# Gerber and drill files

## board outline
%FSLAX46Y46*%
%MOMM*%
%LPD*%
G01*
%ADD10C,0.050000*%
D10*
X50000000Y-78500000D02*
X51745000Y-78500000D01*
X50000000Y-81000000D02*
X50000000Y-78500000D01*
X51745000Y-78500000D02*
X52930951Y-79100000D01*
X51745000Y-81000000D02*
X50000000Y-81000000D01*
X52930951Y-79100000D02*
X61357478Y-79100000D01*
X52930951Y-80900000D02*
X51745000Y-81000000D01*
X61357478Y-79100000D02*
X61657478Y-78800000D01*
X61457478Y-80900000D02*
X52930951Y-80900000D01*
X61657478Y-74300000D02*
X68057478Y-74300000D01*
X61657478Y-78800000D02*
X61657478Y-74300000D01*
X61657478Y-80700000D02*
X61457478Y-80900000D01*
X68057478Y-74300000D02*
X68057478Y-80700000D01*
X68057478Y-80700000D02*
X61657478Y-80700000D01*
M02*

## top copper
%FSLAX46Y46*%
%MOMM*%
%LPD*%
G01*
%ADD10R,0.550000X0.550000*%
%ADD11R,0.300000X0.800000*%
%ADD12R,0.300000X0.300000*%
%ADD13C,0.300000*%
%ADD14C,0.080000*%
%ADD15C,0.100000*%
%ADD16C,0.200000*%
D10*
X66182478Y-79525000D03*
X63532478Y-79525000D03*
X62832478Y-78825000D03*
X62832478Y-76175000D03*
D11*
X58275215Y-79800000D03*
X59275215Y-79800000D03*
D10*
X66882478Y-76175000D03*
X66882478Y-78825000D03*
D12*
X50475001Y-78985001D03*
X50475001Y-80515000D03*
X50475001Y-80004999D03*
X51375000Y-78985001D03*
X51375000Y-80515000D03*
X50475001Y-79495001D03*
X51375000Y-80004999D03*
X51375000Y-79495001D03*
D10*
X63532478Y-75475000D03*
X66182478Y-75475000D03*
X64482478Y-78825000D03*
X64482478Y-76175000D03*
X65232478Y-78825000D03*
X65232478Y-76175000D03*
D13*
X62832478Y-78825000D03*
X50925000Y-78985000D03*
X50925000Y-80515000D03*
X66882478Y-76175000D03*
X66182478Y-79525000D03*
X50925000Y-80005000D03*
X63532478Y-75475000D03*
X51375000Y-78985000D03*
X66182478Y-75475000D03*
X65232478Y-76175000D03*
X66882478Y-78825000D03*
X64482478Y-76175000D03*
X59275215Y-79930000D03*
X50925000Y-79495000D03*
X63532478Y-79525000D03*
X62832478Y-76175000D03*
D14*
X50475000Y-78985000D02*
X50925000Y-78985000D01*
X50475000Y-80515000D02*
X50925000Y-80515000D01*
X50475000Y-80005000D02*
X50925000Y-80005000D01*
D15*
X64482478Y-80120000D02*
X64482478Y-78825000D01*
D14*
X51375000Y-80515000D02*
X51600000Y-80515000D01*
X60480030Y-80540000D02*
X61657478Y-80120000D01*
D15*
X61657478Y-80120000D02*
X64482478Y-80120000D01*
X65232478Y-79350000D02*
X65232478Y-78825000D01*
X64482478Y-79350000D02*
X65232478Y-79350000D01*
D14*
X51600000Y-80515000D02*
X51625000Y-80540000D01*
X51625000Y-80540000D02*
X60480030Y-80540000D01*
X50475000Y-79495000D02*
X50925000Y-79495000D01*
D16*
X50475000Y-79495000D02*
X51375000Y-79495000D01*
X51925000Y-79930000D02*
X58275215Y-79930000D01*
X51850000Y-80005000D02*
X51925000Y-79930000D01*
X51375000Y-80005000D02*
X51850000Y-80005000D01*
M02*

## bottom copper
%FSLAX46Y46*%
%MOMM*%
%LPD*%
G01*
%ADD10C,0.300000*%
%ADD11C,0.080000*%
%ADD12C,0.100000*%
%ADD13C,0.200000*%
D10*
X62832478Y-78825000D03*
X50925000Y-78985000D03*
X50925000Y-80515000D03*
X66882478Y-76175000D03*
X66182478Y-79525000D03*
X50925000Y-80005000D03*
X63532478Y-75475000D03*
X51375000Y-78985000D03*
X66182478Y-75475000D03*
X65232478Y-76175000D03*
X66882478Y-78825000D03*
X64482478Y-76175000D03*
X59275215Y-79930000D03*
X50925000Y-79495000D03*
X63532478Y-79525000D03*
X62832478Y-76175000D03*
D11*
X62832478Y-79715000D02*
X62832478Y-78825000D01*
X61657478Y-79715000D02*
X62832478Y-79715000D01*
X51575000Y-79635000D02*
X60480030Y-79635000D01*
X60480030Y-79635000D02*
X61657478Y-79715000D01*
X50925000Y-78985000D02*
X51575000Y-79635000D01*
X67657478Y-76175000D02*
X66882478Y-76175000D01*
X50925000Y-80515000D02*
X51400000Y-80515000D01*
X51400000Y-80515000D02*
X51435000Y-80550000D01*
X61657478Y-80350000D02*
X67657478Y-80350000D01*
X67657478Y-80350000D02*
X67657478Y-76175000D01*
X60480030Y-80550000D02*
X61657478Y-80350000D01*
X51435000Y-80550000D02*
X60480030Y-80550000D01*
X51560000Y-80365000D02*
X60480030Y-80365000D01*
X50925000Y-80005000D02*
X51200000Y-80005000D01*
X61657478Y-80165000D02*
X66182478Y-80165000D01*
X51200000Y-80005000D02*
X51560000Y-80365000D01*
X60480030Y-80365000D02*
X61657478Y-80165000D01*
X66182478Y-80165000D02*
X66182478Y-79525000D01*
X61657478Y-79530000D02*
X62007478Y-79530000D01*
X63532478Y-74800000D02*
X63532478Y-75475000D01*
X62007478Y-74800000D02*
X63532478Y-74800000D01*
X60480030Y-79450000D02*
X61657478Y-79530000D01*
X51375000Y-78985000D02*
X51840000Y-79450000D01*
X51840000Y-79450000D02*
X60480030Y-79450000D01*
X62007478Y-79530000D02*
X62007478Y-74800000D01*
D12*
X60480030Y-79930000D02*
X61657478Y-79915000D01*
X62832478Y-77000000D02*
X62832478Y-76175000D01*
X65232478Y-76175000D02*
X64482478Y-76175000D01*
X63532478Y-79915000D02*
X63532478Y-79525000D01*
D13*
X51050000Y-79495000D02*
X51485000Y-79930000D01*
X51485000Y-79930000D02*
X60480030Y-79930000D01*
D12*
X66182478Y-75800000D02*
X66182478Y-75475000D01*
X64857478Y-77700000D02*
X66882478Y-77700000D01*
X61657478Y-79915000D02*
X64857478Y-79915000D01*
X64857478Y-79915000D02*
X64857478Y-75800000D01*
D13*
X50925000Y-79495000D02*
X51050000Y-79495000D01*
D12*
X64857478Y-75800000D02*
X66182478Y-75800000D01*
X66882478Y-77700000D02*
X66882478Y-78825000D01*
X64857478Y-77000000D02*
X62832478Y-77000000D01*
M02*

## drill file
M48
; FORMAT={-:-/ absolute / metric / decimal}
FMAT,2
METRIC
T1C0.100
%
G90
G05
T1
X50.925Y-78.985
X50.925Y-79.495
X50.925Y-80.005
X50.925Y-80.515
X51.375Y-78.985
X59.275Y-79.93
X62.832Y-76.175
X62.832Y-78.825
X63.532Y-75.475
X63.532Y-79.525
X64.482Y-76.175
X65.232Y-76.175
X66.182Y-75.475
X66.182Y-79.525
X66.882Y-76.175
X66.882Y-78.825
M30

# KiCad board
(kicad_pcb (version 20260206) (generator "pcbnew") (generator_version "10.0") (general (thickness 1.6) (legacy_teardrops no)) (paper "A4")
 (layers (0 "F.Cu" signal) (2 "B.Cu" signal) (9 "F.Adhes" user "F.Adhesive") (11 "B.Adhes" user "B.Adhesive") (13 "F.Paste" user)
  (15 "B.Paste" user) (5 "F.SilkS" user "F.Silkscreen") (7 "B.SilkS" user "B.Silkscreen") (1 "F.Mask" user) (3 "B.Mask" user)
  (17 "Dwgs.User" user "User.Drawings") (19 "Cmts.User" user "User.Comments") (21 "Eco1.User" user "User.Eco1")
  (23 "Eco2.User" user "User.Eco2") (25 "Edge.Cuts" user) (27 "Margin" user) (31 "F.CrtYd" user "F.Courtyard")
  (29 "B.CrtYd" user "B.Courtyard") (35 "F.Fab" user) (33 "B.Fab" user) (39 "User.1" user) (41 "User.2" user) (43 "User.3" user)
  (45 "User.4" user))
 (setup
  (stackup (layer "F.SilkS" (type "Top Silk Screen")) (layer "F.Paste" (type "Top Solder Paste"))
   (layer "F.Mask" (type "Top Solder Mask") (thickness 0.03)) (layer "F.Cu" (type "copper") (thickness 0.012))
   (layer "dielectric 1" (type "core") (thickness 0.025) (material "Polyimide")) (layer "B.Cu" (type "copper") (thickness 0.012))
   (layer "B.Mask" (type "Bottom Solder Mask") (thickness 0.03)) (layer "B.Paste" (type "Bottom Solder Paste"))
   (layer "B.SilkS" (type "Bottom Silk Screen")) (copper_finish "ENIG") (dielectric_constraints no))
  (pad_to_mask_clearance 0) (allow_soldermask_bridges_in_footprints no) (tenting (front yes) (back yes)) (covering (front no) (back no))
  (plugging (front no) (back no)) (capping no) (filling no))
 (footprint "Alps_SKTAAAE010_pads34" (layer "F.Cu") (at 64.857478 75.1)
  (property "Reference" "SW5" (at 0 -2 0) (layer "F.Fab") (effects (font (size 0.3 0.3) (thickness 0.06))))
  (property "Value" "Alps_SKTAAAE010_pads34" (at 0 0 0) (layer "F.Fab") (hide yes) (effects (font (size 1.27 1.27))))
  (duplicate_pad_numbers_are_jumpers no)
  (pad "3" smd rect (at -1.325 0.375) (size 0.55 0.55) (layers "F.Cu" "F.Mask" "F.Paste") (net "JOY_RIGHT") (solder_mask_margin 0.05)
   (thermal_bridge_angle 45))
  (pad "4" smd rect (at 1.325 0.375) (size 0.55 0.55) (layers "F.Cu" "F.Mask" "F.Paste") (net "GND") (solder_mask_margin 0.05)
   (thermal_bridge_angle 45)))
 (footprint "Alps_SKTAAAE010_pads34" (layer "F.Cu") (at 62.457478 77.5 90)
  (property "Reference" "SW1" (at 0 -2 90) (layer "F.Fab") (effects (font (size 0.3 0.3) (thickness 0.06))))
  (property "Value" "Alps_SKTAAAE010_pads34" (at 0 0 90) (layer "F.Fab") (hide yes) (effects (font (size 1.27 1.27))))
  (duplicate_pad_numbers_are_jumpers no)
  (pad "3" smd rect (at -1.325 0.375 90) (size 0.55 0.55) (layers "F.Cu" "F.Mask" "F.Paste") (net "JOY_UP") (solder_mask_margin 0.05)
   (thermal_bridge_angle 45))
  (pad "4" smd rect (at 1.325 0.375 90) (size 0.55 0.55) (layers "F.Cu" "F.Mask" "F.Paste") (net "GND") (solder_mask_margin 0.05)
   (thermal_bridge_angle 45)))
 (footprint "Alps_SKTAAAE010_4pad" (layer "F.Cu") (at 64.857478 77.5 90)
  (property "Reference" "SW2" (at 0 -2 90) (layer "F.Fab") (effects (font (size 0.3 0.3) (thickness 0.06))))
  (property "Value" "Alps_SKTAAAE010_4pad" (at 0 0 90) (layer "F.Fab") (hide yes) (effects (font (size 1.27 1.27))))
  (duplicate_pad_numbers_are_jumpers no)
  (pad "1" smd rect (at -1.325 -0.375 90) (size 0.55 0.55) (layers "F.Cu" "F.Mask" "F.Paste") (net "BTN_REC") (solder_mask_margin 0.05)
   (thermal_bridge_angle 45))
  (pad "2" smd rect (at 1.325 -0.375 90) (size 0.55 0.55) (layers "F.Cu" "F.Mask" "F.Paste") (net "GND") (solder_mask_margin 0.05)
   (thermal_bridge_angle 45))
  (pad "3" smd rect (at -1.325 0.375 90) (size 0.55 0.55) (layers "F.Cu" "F.Mask" "F.Paste") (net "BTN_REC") (solder_mask_margin 0.05)
   (thermal_bridge_angle 45))
  (pad "4" smd rect (at 1.325 0.375 90) (size 0.55 0.55) (layers "F.Cu" "F.Mask" "F.Paste") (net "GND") (solder_mask_margin 0.05)
   (thermal_bridge_angle 45)))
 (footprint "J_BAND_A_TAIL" (layer "F.Cu") (at 50.9 79.75)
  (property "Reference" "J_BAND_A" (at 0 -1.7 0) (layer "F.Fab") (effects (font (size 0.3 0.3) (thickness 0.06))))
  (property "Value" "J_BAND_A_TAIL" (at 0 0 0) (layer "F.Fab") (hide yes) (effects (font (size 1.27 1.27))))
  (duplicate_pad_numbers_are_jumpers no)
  (pad "1" smd rect (at -0.424999 -0.764999) (size 0.3 0.3) (layers "F.Cu" "F.Mask") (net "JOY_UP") (solder_mask_margin 0.05)
   (thermal_bridge_angle 45))
  (pad "2" smd rect (at -0.424999 0.765) (size 0.3 0.3) (layers "F.Cu" "F.Mask") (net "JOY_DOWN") (solder_mask_margin 0.05)
   (thermal_bridge_angle 45))
  (pad "3" smd rect (at -0.424999 0.254999) (size 0.3 0.3) (layers "F.Cu" "F.Mask") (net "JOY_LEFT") (solder_mask_margin 0.05)
   (thermal_bridge_angle 45))
  (pad "4" smd rect (at 0.475 -0.764999) (size 0.3 0.3) (layers "F.Cu" "F.Mask") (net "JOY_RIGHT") (solder_mask_margin 0.05)
   (thermal_bridge_angle 45))
  (pad "5" smd rect (at 0.475 0.765) (size 0.3 0.3) (layers "F.Cu" "F.Mask") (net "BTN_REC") (solder_mask_margin 0.05)
   (thermal_bridge_angle 45))
  (pad "6" smd rect (at -0.424999 -0.254999) (size 0.3 0.3) (layers "F.Cu" "F.Mask") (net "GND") (solder_mask_margin 0.05)
   (thermal_bridge_angle 45))
  (pad "7" smd rect (at 0.475 0.254999) (size 0.3 0.3) (layers "F.Cu" "F.Mask") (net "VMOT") (solder_mask_margin 0.05)
   (thermal_bridge_angle 45))
  (pad "8" smd rect (at 0.475 -0.254999) (size 0.3 0.3) (layers "F.Cu" "F.Mask") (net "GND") (solder_mask_margin 0.05)
   (thermal_bridge_angle 45)))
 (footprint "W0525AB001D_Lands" (layer "F.Cu") (at 58.775215 79.93)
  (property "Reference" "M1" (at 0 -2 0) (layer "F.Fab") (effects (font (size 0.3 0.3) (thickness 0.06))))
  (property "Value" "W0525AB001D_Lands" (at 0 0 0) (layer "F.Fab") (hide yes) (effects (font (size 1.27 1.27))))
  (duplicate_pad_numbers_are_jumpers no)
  (pad "1" smd rect (at -0.5 -0.13) (size 0.3 0.8) (layers "F.Cu" "F.Mask") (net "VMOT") (solder_mask_margin 0.05) (thermal_bridge_angle 45))
  (pad "2" smd rect (at 0.5 -0.13) (size 0.3 0.8) (layers "F.Cu" "F.Mask") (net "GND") (solder_mask_margin 0.05) (thermal_bridge_angle 45)))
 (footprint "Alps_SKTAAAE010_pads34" (layer "F.Cu") (at 64.857478 79.9 180)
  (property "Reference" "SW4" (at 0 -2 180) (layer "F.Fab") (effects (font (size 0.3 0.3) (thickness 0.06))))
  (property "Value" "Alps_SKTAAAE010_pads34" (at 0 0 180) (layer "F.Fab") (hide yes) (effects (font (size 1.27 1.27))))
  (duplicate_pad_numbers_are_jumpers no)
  (pad "3" smd rect (at -1.325 0.375 180) (size 0.55 0.55) (layers "F.Cu" "F.Mask" "F.Paste") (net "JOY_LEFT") (solder_mask_margin 0.05)
   (thermal_bridge_angle 45))
  (pad "4" smd rect (at 1.325 0.375 180) (size 0.55 0.55) (layers "F.Cu" "F.Mask" "F.Paste") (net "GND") (solder_mask_margin 0.05)
   (thermal_bridge_angle 45)))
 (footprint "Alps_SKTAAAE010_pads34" (layer "F.Cu") (at 67.257478 77.5 -90)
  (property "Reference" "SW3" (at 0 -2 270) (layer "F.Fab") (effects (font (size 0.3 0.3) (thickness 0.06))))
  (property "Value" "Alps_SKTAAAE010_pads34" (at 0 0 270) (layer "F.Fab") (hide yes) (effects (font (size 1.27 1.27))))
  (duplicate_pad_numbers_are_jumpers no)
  (pad "3" smd rect (at -1.325 0.375 270) (size 0.55 0.55) (layers "F.Cu" "F.Mask" "F.Paste") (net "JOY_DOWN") (solder_mask_margin 0.05)
   (thermal_bridge_angle 45))
  (pad "4" smd rect (at 1.325 0.375 270) (size 0.55 0.55) (layers "F.Cu" "F.Mask" "F.Paste") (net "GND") (solder_mask_margin 0.05)
   (thermal_bridge_angle 45)))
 (gr_line (start 50 78.5) (end 51.745 78.5) (stroke (width 0.05) (type default)) (layer "Edge.Cuts"))
 (gr_line (start 50 81) (end 50 78.5) (stroke (width 0.05) (type default)) (layer "Edge.Cuts"))
 (gr_line (start 51.745 78.5) (end 52.930951 79.1) (stroke (width 0.05) (type default)) (layer "Edge.Cuts"))
 (gr_line (start 51.745 81) (end 50 81) (stroke (width 0.05) (type default)) (layer "Edge.Cuts"))
 (gr_line (start 52.930951 79.1) (end 61.357478 79.1) (stroke (width 0.05) (type default)) (layer "Edge.Cuts"))
 (gr_line (start 52.930951 80.9) (end 51.745 81) (stroke (width 0.05) (type default)) (layer "Edge.Cuts"))
 (gr_line (start 61.357478 79.1) (end 61.657478 78.8) (stroke (width 0.05) (type default)) (layer "Edge.Cuts"))
 (gr_line (start 61.457478 80.9) (end 52.930951 80.9) (stroke (width 0.05) (type default)) (layer "Edge.Cuts"))
 (gr_line (start 61.657478 74.3) (end 68.057478 74.3) (stroke (width 0.05) (type default)) (layer "Edge.Cuts"))
 (gr_line (start 61.657478 78.8) (end 61.657478 74.3) (stroke (width 0.05) (type default)) (layer "Edge.Cuts"))
 (gr_line (start 61.657478 80.7) (end 61.457478 80.9) (stroke (width 0.05) (type default)) (layer "Edge.Cuts"))
 (gr_line (start 68.057478 74.3) (end 68.057478 80.7) (stroke (width 0.05) (type default)) (layer "Edge.Cuts"))
 (gr_line (start 68.057478 80.7) (end 61.657478 80.7) (stroke (width 0.05) (type default)) (layer "Edge.Cuts"))
 (segment (start 50.475 78.985) (end 50.925 78.985) (width 0.08) (layer "F.Cu") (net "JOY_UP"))
 (via (at 50.925 78.985) (size 0.3) (drill 0.1) (layers "F.Cu" "B.Cu") (tenting (front yes) (back yes)) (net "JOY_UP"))
 (via (at 62.832478 78.825) (size 0.3) (drill 0.1) (layers "F.Cu" "B.Cu") (tenting (front yes) (back yes)) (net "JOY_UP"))
 (segment (start 60.48003 79.635) (end 61.657478 79.715) (width 0.08) (layer "B.Cu") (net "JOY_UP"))
 (segment (start 61.657478 79.715) (end 62.832478 79.715) (width 0.08) (layer "B.Cu") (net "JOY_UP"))
 (segment (start 50.925 78.985) (end 51.575 79.635) (width 0.08) (layer "B.Cu") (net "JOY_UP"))
 (segment (start 62.832478 79.715) (end 62.832478 78.825) (width 0.08) (layer "B.Cu") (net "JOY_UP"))
 (segment (start 51.575 79.635) (end 60.48003 79.635) (width 0.08) (layer "B.Cu") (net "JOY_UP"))
 (segment (start 50.475 80.515) (end 50.925 80.515) (width 0.08) (layer "F.Cu") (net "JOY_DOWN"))
 (via (at 50.925 80.515) (size 0.3) (drill 0.1) (layers "F.Cu" "B.Cu") (tenting (front yes) (back yes)) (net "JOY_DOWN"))
 (via (at 66.882478 76.175) (size 0.3) (drill 0.1) (layers "F.Cu" "B.Cu") (tenting (front yes) (back yes)) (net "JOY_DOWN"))
 (segment (start 50.925 80.515) (end 51.4 80.515) (width 0.08) (layer "B.Cu") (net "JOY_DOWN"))
 (segment (start 67.657478 80.35) (end 67.657478 76.175) (width 0.08) (layer "B.Cu") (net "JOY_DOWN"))
 (segment (start 60.48003 80.55) (end 61.657478 80.35) (width 0.08) (layer "B.Cu") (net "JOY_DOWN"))
 (segment (start 67.657478 76.175) (end 66.882478 76.175) (width 0.08) (layer "B.Cu") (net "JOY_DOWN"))
 (segment (start 51.435 80.55) (end 60.48003 80.55) (width 0.08) (layer "B.Cu") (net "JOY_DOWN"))
 (segment (start 51.4 80.515) (end 51.435 80.55) (width 0.08) (layer "B.Cu") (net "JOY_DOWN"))
 (segment (start 61.657478 80.35) (end 67.657478 80.35) (width 0.08) (layer "B.Cu") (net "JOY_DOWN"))
 (segment (start 50.475 80.005) (end 50.925 80.005) (width 0.08) (layer "F.Cu") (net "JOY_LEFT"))
 (via (at 66.182478 79.525) (size 0.3) (drill 0.1) (layers "F.Cu" "B.Cu") (tenting (front yes) (back yes)) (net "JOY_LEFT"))
 (via (at 50.925 80.005) (size 0.3) (drill 0.1) (layers "F.Cu" "B.Cu") (tenting (front yes) (back yes)) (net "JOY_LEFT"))
 (segment (start 51.56 80.365) (end 60.48003 80.365) (width 0.08) (layer "B.Cu") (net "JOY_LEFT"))
 (segment (start 61.657478 80.165) (end 66.182478 80.165) (width 0.08) (layer "B.Cu") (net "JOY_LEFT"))
 (segment (start 51.2 80.005) (end 51.56 80.365) (width 0.08) (layer "B.Cu") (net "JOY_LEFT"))
 (segment (start 60.48003 80.365) (end 61.657478 80.165) (width 0.08) (layer "B.Cu") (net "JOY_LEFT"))
 (segment (start 66.182478 80.165) (end 66.182478 79.525) (width 0.08) (layer "B.Cu") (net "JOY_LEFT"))
 (segment (start 50.925 80.005) (end 51.2 80.005) (width 0.08) (layer "B.Cu") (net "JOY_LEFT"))
 (via (at 63.532478 75.475) (size 0.3) (drill 0.1) (layers "F.Cu" "B.Cu") (tenting (front yes) (back yes)) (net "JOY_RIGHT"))
 (via (at 51.375 78.985) (size 0.3) (drill 0.1) (layers "F.Cu" "B.Cu") (tenting (front yes) (back yes)) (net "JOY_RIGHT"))
 (segment (start 62.007478 74.8) (end 63.532478 74.8) (width 0.08) (layer "B.Cu") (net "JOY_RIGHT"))
 (segment (start 60.48003 79.45) (end 61.657478 79.53) (width 0.08) (layer "B.Cu") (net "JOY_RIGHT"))
 (segment (start 51.84 79.45) (end 60.48003 79.45) (width 0.08) (layer "B.Cu") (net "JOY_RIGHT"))
 (segment (start 63.532478 74.8) (end 63.532478 75.475) (width 0.08) (layer "B.Cu") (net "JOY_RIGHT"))
 (segment (start 62.007478 79.53) (end 62.007478 74.8) (width 0.08) (layer "B.Cu") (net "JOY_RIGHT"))
 (segment (start 61.657478 79.53) (end 62.007478 79.53) (width 0.08) (layer "B.Cu") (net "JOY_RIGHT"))
 (segment (start 51.375 78.985) (end 51.84 79.45) (width 0.08) (layer "B.Cu") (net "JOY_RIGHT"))
 (segment (start 61.657478 80.12) (end 64.482478 80.12) (width 0.1) (layer "F.Cu") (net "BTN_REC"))
 (segment (start 60.48003 80.54) (end 61.657478 80.12) (width 0.08) (layer "F.Cu") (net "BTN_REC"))
 (segment (start 51.625 80.54) (end 60.48003 80.54) (width 0.08) (layer "F.Cu") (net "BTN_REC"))
 (segment (start 51.6 80.515) (end 51.625 80.54) (width 0.08) (layer "F.Cu") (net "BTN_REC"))
 (segment (start 64.482478 79.35) (end 65.232478 79.35) (width 0.1) (layer "F.Cu") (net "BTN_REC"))
 (segment (start 64.482478 80.12) (end 64.482478 78.825) (width 0.1) (layer "F.Cu") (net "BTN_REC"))
 (segment (start 65.232478 79.35) (end 65.232478 78.825) (width 0.1) (layer "F.Cu") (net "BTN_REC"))
 (segment (start 51.375 80.515) (end 51.6 80.515) (width 0.08) (layer "F.Cu") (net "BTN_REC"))
 (segment (start 50.475 79.495) (end 50.925 79.495) (width 0.08) (layer "F.Cu") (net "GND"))
 (segment (start 50.475 79.495) (end 51.375 79.495) (width 0.2) (layer "F.Cu") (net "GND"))
 (via (at 50.925 79.495) (size 0.3) (drill 0.1) (layers "F.Cu" "B.Cu") (tenting (front yes) (back yes)) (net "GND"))
 (via (at 59.275215 79.93) (size 0.3) (drill 0.1) (layers "F.Cu" "B.Cu") (tenting (front yes) (back yes)) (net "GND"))
 (via (at 63.532478 79.525) (size 0.3) (drill 0.1) (layers "F.Cu" "B.Cu") (tenting (front yes) (back yes)) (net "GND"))
 (via (at 66.182478 75.475) (size 0.3) (drill 0.1) (layers "F.Cu" "B.Cu") (tenting (front yes) (back yes)) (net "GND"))
 (via (at 64.482478 76.175) (size 0.3) (drill 0.1) (layers "F.Cu" "B.Cu") (tenting (front yes) (back yes)) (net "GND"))
 (via (at 62.832478 76.175) (size 0.3) (drill 0.1) (layers "F.Cu" "B.Cu") (tenting (front yes) (back yes)) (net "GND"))
 (via (at 65.232478 76.175) (size 0.3) (drill 0.1) (layers "F.Cu" "B.Cu") (tenting (front yes) (back yes)) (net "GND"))
 (via (at 66.882478 78.825) (size 0.3) (drill 0.1) (layers "F.Cu" "B.Cu") (tenting (front yes) (back yes)) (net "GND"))
 (segment (start 51.05 79.495) (end 51.485 79.93) (width 0.2) (layer "B.Cu") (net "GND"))
 (segment (start 66.882478 77.7) (end 66.882478 78.825) (width 0.1) (layer "B.Cu") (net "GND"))
 (segment (start 50.925 79.495) (end 51.05 79.495) (width 0.2) (layer "B.Cu") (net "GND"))
 (segment (start 64.857478 79.915) (end 64.857478 75.8) (width 0.1) (layer "B.Cu") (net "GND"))
 (segment (start 51.485 79.93) (end 60.48003 79.93) (width 0.2) (layer "B.Cu") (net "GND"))
 (segment (start 64.857478 77) (end 62.832478 77) (width 0.1) (layer "B.Cu") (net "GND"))
 (segment (start 64.857478 77.7) (end 66.882478 77.7) (width 0.1) (layer "B.Cu") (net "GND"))
 (segment (start 64.857478 75.8) (end 66.182478 75.8) (width 0.1) (layer "B.Cu") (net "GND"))
 (segment (start 60.48003 79.93) (end 61.657478 79.915) (width 0.1) (layer "B.Cu") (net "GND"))
 (segment (start 62.832478 77) (end 62.832478 76.175) (width 0.1) (layer "B.Cu") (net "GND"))
 (segment (start 65.232478 76.175) (end 64.482478 76.175) (width 0.1) (layer "B.Cu") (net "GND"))
 (segment (start 63.532478 79.915) (end 63.532478 79.525) (width 0.1) (layer "B.Cu") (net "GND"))
 (segment (start 61.657478 79.915) (end 64.857478 79.915) (width 0.1) (layer "B.Cu") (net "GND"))
 (segment (start 66.182478 75.8) (end 66.182478 75.475) (width 0.1) (layer "B.Cu") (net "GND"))
 (segment (start 51.375 80.005) (end 51.85 80.005) (width 0.2) (layer "F.Cu") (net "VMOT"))
 (segment (start 51.925 79.93) (end 58.275215 79.93) (width 0.2) (layer "F.Cu") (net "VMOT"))
 (segment (start 51.85 80.005) (end 51.925 79.93) (width 0.2) (layer "F.Cu") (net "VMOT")))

